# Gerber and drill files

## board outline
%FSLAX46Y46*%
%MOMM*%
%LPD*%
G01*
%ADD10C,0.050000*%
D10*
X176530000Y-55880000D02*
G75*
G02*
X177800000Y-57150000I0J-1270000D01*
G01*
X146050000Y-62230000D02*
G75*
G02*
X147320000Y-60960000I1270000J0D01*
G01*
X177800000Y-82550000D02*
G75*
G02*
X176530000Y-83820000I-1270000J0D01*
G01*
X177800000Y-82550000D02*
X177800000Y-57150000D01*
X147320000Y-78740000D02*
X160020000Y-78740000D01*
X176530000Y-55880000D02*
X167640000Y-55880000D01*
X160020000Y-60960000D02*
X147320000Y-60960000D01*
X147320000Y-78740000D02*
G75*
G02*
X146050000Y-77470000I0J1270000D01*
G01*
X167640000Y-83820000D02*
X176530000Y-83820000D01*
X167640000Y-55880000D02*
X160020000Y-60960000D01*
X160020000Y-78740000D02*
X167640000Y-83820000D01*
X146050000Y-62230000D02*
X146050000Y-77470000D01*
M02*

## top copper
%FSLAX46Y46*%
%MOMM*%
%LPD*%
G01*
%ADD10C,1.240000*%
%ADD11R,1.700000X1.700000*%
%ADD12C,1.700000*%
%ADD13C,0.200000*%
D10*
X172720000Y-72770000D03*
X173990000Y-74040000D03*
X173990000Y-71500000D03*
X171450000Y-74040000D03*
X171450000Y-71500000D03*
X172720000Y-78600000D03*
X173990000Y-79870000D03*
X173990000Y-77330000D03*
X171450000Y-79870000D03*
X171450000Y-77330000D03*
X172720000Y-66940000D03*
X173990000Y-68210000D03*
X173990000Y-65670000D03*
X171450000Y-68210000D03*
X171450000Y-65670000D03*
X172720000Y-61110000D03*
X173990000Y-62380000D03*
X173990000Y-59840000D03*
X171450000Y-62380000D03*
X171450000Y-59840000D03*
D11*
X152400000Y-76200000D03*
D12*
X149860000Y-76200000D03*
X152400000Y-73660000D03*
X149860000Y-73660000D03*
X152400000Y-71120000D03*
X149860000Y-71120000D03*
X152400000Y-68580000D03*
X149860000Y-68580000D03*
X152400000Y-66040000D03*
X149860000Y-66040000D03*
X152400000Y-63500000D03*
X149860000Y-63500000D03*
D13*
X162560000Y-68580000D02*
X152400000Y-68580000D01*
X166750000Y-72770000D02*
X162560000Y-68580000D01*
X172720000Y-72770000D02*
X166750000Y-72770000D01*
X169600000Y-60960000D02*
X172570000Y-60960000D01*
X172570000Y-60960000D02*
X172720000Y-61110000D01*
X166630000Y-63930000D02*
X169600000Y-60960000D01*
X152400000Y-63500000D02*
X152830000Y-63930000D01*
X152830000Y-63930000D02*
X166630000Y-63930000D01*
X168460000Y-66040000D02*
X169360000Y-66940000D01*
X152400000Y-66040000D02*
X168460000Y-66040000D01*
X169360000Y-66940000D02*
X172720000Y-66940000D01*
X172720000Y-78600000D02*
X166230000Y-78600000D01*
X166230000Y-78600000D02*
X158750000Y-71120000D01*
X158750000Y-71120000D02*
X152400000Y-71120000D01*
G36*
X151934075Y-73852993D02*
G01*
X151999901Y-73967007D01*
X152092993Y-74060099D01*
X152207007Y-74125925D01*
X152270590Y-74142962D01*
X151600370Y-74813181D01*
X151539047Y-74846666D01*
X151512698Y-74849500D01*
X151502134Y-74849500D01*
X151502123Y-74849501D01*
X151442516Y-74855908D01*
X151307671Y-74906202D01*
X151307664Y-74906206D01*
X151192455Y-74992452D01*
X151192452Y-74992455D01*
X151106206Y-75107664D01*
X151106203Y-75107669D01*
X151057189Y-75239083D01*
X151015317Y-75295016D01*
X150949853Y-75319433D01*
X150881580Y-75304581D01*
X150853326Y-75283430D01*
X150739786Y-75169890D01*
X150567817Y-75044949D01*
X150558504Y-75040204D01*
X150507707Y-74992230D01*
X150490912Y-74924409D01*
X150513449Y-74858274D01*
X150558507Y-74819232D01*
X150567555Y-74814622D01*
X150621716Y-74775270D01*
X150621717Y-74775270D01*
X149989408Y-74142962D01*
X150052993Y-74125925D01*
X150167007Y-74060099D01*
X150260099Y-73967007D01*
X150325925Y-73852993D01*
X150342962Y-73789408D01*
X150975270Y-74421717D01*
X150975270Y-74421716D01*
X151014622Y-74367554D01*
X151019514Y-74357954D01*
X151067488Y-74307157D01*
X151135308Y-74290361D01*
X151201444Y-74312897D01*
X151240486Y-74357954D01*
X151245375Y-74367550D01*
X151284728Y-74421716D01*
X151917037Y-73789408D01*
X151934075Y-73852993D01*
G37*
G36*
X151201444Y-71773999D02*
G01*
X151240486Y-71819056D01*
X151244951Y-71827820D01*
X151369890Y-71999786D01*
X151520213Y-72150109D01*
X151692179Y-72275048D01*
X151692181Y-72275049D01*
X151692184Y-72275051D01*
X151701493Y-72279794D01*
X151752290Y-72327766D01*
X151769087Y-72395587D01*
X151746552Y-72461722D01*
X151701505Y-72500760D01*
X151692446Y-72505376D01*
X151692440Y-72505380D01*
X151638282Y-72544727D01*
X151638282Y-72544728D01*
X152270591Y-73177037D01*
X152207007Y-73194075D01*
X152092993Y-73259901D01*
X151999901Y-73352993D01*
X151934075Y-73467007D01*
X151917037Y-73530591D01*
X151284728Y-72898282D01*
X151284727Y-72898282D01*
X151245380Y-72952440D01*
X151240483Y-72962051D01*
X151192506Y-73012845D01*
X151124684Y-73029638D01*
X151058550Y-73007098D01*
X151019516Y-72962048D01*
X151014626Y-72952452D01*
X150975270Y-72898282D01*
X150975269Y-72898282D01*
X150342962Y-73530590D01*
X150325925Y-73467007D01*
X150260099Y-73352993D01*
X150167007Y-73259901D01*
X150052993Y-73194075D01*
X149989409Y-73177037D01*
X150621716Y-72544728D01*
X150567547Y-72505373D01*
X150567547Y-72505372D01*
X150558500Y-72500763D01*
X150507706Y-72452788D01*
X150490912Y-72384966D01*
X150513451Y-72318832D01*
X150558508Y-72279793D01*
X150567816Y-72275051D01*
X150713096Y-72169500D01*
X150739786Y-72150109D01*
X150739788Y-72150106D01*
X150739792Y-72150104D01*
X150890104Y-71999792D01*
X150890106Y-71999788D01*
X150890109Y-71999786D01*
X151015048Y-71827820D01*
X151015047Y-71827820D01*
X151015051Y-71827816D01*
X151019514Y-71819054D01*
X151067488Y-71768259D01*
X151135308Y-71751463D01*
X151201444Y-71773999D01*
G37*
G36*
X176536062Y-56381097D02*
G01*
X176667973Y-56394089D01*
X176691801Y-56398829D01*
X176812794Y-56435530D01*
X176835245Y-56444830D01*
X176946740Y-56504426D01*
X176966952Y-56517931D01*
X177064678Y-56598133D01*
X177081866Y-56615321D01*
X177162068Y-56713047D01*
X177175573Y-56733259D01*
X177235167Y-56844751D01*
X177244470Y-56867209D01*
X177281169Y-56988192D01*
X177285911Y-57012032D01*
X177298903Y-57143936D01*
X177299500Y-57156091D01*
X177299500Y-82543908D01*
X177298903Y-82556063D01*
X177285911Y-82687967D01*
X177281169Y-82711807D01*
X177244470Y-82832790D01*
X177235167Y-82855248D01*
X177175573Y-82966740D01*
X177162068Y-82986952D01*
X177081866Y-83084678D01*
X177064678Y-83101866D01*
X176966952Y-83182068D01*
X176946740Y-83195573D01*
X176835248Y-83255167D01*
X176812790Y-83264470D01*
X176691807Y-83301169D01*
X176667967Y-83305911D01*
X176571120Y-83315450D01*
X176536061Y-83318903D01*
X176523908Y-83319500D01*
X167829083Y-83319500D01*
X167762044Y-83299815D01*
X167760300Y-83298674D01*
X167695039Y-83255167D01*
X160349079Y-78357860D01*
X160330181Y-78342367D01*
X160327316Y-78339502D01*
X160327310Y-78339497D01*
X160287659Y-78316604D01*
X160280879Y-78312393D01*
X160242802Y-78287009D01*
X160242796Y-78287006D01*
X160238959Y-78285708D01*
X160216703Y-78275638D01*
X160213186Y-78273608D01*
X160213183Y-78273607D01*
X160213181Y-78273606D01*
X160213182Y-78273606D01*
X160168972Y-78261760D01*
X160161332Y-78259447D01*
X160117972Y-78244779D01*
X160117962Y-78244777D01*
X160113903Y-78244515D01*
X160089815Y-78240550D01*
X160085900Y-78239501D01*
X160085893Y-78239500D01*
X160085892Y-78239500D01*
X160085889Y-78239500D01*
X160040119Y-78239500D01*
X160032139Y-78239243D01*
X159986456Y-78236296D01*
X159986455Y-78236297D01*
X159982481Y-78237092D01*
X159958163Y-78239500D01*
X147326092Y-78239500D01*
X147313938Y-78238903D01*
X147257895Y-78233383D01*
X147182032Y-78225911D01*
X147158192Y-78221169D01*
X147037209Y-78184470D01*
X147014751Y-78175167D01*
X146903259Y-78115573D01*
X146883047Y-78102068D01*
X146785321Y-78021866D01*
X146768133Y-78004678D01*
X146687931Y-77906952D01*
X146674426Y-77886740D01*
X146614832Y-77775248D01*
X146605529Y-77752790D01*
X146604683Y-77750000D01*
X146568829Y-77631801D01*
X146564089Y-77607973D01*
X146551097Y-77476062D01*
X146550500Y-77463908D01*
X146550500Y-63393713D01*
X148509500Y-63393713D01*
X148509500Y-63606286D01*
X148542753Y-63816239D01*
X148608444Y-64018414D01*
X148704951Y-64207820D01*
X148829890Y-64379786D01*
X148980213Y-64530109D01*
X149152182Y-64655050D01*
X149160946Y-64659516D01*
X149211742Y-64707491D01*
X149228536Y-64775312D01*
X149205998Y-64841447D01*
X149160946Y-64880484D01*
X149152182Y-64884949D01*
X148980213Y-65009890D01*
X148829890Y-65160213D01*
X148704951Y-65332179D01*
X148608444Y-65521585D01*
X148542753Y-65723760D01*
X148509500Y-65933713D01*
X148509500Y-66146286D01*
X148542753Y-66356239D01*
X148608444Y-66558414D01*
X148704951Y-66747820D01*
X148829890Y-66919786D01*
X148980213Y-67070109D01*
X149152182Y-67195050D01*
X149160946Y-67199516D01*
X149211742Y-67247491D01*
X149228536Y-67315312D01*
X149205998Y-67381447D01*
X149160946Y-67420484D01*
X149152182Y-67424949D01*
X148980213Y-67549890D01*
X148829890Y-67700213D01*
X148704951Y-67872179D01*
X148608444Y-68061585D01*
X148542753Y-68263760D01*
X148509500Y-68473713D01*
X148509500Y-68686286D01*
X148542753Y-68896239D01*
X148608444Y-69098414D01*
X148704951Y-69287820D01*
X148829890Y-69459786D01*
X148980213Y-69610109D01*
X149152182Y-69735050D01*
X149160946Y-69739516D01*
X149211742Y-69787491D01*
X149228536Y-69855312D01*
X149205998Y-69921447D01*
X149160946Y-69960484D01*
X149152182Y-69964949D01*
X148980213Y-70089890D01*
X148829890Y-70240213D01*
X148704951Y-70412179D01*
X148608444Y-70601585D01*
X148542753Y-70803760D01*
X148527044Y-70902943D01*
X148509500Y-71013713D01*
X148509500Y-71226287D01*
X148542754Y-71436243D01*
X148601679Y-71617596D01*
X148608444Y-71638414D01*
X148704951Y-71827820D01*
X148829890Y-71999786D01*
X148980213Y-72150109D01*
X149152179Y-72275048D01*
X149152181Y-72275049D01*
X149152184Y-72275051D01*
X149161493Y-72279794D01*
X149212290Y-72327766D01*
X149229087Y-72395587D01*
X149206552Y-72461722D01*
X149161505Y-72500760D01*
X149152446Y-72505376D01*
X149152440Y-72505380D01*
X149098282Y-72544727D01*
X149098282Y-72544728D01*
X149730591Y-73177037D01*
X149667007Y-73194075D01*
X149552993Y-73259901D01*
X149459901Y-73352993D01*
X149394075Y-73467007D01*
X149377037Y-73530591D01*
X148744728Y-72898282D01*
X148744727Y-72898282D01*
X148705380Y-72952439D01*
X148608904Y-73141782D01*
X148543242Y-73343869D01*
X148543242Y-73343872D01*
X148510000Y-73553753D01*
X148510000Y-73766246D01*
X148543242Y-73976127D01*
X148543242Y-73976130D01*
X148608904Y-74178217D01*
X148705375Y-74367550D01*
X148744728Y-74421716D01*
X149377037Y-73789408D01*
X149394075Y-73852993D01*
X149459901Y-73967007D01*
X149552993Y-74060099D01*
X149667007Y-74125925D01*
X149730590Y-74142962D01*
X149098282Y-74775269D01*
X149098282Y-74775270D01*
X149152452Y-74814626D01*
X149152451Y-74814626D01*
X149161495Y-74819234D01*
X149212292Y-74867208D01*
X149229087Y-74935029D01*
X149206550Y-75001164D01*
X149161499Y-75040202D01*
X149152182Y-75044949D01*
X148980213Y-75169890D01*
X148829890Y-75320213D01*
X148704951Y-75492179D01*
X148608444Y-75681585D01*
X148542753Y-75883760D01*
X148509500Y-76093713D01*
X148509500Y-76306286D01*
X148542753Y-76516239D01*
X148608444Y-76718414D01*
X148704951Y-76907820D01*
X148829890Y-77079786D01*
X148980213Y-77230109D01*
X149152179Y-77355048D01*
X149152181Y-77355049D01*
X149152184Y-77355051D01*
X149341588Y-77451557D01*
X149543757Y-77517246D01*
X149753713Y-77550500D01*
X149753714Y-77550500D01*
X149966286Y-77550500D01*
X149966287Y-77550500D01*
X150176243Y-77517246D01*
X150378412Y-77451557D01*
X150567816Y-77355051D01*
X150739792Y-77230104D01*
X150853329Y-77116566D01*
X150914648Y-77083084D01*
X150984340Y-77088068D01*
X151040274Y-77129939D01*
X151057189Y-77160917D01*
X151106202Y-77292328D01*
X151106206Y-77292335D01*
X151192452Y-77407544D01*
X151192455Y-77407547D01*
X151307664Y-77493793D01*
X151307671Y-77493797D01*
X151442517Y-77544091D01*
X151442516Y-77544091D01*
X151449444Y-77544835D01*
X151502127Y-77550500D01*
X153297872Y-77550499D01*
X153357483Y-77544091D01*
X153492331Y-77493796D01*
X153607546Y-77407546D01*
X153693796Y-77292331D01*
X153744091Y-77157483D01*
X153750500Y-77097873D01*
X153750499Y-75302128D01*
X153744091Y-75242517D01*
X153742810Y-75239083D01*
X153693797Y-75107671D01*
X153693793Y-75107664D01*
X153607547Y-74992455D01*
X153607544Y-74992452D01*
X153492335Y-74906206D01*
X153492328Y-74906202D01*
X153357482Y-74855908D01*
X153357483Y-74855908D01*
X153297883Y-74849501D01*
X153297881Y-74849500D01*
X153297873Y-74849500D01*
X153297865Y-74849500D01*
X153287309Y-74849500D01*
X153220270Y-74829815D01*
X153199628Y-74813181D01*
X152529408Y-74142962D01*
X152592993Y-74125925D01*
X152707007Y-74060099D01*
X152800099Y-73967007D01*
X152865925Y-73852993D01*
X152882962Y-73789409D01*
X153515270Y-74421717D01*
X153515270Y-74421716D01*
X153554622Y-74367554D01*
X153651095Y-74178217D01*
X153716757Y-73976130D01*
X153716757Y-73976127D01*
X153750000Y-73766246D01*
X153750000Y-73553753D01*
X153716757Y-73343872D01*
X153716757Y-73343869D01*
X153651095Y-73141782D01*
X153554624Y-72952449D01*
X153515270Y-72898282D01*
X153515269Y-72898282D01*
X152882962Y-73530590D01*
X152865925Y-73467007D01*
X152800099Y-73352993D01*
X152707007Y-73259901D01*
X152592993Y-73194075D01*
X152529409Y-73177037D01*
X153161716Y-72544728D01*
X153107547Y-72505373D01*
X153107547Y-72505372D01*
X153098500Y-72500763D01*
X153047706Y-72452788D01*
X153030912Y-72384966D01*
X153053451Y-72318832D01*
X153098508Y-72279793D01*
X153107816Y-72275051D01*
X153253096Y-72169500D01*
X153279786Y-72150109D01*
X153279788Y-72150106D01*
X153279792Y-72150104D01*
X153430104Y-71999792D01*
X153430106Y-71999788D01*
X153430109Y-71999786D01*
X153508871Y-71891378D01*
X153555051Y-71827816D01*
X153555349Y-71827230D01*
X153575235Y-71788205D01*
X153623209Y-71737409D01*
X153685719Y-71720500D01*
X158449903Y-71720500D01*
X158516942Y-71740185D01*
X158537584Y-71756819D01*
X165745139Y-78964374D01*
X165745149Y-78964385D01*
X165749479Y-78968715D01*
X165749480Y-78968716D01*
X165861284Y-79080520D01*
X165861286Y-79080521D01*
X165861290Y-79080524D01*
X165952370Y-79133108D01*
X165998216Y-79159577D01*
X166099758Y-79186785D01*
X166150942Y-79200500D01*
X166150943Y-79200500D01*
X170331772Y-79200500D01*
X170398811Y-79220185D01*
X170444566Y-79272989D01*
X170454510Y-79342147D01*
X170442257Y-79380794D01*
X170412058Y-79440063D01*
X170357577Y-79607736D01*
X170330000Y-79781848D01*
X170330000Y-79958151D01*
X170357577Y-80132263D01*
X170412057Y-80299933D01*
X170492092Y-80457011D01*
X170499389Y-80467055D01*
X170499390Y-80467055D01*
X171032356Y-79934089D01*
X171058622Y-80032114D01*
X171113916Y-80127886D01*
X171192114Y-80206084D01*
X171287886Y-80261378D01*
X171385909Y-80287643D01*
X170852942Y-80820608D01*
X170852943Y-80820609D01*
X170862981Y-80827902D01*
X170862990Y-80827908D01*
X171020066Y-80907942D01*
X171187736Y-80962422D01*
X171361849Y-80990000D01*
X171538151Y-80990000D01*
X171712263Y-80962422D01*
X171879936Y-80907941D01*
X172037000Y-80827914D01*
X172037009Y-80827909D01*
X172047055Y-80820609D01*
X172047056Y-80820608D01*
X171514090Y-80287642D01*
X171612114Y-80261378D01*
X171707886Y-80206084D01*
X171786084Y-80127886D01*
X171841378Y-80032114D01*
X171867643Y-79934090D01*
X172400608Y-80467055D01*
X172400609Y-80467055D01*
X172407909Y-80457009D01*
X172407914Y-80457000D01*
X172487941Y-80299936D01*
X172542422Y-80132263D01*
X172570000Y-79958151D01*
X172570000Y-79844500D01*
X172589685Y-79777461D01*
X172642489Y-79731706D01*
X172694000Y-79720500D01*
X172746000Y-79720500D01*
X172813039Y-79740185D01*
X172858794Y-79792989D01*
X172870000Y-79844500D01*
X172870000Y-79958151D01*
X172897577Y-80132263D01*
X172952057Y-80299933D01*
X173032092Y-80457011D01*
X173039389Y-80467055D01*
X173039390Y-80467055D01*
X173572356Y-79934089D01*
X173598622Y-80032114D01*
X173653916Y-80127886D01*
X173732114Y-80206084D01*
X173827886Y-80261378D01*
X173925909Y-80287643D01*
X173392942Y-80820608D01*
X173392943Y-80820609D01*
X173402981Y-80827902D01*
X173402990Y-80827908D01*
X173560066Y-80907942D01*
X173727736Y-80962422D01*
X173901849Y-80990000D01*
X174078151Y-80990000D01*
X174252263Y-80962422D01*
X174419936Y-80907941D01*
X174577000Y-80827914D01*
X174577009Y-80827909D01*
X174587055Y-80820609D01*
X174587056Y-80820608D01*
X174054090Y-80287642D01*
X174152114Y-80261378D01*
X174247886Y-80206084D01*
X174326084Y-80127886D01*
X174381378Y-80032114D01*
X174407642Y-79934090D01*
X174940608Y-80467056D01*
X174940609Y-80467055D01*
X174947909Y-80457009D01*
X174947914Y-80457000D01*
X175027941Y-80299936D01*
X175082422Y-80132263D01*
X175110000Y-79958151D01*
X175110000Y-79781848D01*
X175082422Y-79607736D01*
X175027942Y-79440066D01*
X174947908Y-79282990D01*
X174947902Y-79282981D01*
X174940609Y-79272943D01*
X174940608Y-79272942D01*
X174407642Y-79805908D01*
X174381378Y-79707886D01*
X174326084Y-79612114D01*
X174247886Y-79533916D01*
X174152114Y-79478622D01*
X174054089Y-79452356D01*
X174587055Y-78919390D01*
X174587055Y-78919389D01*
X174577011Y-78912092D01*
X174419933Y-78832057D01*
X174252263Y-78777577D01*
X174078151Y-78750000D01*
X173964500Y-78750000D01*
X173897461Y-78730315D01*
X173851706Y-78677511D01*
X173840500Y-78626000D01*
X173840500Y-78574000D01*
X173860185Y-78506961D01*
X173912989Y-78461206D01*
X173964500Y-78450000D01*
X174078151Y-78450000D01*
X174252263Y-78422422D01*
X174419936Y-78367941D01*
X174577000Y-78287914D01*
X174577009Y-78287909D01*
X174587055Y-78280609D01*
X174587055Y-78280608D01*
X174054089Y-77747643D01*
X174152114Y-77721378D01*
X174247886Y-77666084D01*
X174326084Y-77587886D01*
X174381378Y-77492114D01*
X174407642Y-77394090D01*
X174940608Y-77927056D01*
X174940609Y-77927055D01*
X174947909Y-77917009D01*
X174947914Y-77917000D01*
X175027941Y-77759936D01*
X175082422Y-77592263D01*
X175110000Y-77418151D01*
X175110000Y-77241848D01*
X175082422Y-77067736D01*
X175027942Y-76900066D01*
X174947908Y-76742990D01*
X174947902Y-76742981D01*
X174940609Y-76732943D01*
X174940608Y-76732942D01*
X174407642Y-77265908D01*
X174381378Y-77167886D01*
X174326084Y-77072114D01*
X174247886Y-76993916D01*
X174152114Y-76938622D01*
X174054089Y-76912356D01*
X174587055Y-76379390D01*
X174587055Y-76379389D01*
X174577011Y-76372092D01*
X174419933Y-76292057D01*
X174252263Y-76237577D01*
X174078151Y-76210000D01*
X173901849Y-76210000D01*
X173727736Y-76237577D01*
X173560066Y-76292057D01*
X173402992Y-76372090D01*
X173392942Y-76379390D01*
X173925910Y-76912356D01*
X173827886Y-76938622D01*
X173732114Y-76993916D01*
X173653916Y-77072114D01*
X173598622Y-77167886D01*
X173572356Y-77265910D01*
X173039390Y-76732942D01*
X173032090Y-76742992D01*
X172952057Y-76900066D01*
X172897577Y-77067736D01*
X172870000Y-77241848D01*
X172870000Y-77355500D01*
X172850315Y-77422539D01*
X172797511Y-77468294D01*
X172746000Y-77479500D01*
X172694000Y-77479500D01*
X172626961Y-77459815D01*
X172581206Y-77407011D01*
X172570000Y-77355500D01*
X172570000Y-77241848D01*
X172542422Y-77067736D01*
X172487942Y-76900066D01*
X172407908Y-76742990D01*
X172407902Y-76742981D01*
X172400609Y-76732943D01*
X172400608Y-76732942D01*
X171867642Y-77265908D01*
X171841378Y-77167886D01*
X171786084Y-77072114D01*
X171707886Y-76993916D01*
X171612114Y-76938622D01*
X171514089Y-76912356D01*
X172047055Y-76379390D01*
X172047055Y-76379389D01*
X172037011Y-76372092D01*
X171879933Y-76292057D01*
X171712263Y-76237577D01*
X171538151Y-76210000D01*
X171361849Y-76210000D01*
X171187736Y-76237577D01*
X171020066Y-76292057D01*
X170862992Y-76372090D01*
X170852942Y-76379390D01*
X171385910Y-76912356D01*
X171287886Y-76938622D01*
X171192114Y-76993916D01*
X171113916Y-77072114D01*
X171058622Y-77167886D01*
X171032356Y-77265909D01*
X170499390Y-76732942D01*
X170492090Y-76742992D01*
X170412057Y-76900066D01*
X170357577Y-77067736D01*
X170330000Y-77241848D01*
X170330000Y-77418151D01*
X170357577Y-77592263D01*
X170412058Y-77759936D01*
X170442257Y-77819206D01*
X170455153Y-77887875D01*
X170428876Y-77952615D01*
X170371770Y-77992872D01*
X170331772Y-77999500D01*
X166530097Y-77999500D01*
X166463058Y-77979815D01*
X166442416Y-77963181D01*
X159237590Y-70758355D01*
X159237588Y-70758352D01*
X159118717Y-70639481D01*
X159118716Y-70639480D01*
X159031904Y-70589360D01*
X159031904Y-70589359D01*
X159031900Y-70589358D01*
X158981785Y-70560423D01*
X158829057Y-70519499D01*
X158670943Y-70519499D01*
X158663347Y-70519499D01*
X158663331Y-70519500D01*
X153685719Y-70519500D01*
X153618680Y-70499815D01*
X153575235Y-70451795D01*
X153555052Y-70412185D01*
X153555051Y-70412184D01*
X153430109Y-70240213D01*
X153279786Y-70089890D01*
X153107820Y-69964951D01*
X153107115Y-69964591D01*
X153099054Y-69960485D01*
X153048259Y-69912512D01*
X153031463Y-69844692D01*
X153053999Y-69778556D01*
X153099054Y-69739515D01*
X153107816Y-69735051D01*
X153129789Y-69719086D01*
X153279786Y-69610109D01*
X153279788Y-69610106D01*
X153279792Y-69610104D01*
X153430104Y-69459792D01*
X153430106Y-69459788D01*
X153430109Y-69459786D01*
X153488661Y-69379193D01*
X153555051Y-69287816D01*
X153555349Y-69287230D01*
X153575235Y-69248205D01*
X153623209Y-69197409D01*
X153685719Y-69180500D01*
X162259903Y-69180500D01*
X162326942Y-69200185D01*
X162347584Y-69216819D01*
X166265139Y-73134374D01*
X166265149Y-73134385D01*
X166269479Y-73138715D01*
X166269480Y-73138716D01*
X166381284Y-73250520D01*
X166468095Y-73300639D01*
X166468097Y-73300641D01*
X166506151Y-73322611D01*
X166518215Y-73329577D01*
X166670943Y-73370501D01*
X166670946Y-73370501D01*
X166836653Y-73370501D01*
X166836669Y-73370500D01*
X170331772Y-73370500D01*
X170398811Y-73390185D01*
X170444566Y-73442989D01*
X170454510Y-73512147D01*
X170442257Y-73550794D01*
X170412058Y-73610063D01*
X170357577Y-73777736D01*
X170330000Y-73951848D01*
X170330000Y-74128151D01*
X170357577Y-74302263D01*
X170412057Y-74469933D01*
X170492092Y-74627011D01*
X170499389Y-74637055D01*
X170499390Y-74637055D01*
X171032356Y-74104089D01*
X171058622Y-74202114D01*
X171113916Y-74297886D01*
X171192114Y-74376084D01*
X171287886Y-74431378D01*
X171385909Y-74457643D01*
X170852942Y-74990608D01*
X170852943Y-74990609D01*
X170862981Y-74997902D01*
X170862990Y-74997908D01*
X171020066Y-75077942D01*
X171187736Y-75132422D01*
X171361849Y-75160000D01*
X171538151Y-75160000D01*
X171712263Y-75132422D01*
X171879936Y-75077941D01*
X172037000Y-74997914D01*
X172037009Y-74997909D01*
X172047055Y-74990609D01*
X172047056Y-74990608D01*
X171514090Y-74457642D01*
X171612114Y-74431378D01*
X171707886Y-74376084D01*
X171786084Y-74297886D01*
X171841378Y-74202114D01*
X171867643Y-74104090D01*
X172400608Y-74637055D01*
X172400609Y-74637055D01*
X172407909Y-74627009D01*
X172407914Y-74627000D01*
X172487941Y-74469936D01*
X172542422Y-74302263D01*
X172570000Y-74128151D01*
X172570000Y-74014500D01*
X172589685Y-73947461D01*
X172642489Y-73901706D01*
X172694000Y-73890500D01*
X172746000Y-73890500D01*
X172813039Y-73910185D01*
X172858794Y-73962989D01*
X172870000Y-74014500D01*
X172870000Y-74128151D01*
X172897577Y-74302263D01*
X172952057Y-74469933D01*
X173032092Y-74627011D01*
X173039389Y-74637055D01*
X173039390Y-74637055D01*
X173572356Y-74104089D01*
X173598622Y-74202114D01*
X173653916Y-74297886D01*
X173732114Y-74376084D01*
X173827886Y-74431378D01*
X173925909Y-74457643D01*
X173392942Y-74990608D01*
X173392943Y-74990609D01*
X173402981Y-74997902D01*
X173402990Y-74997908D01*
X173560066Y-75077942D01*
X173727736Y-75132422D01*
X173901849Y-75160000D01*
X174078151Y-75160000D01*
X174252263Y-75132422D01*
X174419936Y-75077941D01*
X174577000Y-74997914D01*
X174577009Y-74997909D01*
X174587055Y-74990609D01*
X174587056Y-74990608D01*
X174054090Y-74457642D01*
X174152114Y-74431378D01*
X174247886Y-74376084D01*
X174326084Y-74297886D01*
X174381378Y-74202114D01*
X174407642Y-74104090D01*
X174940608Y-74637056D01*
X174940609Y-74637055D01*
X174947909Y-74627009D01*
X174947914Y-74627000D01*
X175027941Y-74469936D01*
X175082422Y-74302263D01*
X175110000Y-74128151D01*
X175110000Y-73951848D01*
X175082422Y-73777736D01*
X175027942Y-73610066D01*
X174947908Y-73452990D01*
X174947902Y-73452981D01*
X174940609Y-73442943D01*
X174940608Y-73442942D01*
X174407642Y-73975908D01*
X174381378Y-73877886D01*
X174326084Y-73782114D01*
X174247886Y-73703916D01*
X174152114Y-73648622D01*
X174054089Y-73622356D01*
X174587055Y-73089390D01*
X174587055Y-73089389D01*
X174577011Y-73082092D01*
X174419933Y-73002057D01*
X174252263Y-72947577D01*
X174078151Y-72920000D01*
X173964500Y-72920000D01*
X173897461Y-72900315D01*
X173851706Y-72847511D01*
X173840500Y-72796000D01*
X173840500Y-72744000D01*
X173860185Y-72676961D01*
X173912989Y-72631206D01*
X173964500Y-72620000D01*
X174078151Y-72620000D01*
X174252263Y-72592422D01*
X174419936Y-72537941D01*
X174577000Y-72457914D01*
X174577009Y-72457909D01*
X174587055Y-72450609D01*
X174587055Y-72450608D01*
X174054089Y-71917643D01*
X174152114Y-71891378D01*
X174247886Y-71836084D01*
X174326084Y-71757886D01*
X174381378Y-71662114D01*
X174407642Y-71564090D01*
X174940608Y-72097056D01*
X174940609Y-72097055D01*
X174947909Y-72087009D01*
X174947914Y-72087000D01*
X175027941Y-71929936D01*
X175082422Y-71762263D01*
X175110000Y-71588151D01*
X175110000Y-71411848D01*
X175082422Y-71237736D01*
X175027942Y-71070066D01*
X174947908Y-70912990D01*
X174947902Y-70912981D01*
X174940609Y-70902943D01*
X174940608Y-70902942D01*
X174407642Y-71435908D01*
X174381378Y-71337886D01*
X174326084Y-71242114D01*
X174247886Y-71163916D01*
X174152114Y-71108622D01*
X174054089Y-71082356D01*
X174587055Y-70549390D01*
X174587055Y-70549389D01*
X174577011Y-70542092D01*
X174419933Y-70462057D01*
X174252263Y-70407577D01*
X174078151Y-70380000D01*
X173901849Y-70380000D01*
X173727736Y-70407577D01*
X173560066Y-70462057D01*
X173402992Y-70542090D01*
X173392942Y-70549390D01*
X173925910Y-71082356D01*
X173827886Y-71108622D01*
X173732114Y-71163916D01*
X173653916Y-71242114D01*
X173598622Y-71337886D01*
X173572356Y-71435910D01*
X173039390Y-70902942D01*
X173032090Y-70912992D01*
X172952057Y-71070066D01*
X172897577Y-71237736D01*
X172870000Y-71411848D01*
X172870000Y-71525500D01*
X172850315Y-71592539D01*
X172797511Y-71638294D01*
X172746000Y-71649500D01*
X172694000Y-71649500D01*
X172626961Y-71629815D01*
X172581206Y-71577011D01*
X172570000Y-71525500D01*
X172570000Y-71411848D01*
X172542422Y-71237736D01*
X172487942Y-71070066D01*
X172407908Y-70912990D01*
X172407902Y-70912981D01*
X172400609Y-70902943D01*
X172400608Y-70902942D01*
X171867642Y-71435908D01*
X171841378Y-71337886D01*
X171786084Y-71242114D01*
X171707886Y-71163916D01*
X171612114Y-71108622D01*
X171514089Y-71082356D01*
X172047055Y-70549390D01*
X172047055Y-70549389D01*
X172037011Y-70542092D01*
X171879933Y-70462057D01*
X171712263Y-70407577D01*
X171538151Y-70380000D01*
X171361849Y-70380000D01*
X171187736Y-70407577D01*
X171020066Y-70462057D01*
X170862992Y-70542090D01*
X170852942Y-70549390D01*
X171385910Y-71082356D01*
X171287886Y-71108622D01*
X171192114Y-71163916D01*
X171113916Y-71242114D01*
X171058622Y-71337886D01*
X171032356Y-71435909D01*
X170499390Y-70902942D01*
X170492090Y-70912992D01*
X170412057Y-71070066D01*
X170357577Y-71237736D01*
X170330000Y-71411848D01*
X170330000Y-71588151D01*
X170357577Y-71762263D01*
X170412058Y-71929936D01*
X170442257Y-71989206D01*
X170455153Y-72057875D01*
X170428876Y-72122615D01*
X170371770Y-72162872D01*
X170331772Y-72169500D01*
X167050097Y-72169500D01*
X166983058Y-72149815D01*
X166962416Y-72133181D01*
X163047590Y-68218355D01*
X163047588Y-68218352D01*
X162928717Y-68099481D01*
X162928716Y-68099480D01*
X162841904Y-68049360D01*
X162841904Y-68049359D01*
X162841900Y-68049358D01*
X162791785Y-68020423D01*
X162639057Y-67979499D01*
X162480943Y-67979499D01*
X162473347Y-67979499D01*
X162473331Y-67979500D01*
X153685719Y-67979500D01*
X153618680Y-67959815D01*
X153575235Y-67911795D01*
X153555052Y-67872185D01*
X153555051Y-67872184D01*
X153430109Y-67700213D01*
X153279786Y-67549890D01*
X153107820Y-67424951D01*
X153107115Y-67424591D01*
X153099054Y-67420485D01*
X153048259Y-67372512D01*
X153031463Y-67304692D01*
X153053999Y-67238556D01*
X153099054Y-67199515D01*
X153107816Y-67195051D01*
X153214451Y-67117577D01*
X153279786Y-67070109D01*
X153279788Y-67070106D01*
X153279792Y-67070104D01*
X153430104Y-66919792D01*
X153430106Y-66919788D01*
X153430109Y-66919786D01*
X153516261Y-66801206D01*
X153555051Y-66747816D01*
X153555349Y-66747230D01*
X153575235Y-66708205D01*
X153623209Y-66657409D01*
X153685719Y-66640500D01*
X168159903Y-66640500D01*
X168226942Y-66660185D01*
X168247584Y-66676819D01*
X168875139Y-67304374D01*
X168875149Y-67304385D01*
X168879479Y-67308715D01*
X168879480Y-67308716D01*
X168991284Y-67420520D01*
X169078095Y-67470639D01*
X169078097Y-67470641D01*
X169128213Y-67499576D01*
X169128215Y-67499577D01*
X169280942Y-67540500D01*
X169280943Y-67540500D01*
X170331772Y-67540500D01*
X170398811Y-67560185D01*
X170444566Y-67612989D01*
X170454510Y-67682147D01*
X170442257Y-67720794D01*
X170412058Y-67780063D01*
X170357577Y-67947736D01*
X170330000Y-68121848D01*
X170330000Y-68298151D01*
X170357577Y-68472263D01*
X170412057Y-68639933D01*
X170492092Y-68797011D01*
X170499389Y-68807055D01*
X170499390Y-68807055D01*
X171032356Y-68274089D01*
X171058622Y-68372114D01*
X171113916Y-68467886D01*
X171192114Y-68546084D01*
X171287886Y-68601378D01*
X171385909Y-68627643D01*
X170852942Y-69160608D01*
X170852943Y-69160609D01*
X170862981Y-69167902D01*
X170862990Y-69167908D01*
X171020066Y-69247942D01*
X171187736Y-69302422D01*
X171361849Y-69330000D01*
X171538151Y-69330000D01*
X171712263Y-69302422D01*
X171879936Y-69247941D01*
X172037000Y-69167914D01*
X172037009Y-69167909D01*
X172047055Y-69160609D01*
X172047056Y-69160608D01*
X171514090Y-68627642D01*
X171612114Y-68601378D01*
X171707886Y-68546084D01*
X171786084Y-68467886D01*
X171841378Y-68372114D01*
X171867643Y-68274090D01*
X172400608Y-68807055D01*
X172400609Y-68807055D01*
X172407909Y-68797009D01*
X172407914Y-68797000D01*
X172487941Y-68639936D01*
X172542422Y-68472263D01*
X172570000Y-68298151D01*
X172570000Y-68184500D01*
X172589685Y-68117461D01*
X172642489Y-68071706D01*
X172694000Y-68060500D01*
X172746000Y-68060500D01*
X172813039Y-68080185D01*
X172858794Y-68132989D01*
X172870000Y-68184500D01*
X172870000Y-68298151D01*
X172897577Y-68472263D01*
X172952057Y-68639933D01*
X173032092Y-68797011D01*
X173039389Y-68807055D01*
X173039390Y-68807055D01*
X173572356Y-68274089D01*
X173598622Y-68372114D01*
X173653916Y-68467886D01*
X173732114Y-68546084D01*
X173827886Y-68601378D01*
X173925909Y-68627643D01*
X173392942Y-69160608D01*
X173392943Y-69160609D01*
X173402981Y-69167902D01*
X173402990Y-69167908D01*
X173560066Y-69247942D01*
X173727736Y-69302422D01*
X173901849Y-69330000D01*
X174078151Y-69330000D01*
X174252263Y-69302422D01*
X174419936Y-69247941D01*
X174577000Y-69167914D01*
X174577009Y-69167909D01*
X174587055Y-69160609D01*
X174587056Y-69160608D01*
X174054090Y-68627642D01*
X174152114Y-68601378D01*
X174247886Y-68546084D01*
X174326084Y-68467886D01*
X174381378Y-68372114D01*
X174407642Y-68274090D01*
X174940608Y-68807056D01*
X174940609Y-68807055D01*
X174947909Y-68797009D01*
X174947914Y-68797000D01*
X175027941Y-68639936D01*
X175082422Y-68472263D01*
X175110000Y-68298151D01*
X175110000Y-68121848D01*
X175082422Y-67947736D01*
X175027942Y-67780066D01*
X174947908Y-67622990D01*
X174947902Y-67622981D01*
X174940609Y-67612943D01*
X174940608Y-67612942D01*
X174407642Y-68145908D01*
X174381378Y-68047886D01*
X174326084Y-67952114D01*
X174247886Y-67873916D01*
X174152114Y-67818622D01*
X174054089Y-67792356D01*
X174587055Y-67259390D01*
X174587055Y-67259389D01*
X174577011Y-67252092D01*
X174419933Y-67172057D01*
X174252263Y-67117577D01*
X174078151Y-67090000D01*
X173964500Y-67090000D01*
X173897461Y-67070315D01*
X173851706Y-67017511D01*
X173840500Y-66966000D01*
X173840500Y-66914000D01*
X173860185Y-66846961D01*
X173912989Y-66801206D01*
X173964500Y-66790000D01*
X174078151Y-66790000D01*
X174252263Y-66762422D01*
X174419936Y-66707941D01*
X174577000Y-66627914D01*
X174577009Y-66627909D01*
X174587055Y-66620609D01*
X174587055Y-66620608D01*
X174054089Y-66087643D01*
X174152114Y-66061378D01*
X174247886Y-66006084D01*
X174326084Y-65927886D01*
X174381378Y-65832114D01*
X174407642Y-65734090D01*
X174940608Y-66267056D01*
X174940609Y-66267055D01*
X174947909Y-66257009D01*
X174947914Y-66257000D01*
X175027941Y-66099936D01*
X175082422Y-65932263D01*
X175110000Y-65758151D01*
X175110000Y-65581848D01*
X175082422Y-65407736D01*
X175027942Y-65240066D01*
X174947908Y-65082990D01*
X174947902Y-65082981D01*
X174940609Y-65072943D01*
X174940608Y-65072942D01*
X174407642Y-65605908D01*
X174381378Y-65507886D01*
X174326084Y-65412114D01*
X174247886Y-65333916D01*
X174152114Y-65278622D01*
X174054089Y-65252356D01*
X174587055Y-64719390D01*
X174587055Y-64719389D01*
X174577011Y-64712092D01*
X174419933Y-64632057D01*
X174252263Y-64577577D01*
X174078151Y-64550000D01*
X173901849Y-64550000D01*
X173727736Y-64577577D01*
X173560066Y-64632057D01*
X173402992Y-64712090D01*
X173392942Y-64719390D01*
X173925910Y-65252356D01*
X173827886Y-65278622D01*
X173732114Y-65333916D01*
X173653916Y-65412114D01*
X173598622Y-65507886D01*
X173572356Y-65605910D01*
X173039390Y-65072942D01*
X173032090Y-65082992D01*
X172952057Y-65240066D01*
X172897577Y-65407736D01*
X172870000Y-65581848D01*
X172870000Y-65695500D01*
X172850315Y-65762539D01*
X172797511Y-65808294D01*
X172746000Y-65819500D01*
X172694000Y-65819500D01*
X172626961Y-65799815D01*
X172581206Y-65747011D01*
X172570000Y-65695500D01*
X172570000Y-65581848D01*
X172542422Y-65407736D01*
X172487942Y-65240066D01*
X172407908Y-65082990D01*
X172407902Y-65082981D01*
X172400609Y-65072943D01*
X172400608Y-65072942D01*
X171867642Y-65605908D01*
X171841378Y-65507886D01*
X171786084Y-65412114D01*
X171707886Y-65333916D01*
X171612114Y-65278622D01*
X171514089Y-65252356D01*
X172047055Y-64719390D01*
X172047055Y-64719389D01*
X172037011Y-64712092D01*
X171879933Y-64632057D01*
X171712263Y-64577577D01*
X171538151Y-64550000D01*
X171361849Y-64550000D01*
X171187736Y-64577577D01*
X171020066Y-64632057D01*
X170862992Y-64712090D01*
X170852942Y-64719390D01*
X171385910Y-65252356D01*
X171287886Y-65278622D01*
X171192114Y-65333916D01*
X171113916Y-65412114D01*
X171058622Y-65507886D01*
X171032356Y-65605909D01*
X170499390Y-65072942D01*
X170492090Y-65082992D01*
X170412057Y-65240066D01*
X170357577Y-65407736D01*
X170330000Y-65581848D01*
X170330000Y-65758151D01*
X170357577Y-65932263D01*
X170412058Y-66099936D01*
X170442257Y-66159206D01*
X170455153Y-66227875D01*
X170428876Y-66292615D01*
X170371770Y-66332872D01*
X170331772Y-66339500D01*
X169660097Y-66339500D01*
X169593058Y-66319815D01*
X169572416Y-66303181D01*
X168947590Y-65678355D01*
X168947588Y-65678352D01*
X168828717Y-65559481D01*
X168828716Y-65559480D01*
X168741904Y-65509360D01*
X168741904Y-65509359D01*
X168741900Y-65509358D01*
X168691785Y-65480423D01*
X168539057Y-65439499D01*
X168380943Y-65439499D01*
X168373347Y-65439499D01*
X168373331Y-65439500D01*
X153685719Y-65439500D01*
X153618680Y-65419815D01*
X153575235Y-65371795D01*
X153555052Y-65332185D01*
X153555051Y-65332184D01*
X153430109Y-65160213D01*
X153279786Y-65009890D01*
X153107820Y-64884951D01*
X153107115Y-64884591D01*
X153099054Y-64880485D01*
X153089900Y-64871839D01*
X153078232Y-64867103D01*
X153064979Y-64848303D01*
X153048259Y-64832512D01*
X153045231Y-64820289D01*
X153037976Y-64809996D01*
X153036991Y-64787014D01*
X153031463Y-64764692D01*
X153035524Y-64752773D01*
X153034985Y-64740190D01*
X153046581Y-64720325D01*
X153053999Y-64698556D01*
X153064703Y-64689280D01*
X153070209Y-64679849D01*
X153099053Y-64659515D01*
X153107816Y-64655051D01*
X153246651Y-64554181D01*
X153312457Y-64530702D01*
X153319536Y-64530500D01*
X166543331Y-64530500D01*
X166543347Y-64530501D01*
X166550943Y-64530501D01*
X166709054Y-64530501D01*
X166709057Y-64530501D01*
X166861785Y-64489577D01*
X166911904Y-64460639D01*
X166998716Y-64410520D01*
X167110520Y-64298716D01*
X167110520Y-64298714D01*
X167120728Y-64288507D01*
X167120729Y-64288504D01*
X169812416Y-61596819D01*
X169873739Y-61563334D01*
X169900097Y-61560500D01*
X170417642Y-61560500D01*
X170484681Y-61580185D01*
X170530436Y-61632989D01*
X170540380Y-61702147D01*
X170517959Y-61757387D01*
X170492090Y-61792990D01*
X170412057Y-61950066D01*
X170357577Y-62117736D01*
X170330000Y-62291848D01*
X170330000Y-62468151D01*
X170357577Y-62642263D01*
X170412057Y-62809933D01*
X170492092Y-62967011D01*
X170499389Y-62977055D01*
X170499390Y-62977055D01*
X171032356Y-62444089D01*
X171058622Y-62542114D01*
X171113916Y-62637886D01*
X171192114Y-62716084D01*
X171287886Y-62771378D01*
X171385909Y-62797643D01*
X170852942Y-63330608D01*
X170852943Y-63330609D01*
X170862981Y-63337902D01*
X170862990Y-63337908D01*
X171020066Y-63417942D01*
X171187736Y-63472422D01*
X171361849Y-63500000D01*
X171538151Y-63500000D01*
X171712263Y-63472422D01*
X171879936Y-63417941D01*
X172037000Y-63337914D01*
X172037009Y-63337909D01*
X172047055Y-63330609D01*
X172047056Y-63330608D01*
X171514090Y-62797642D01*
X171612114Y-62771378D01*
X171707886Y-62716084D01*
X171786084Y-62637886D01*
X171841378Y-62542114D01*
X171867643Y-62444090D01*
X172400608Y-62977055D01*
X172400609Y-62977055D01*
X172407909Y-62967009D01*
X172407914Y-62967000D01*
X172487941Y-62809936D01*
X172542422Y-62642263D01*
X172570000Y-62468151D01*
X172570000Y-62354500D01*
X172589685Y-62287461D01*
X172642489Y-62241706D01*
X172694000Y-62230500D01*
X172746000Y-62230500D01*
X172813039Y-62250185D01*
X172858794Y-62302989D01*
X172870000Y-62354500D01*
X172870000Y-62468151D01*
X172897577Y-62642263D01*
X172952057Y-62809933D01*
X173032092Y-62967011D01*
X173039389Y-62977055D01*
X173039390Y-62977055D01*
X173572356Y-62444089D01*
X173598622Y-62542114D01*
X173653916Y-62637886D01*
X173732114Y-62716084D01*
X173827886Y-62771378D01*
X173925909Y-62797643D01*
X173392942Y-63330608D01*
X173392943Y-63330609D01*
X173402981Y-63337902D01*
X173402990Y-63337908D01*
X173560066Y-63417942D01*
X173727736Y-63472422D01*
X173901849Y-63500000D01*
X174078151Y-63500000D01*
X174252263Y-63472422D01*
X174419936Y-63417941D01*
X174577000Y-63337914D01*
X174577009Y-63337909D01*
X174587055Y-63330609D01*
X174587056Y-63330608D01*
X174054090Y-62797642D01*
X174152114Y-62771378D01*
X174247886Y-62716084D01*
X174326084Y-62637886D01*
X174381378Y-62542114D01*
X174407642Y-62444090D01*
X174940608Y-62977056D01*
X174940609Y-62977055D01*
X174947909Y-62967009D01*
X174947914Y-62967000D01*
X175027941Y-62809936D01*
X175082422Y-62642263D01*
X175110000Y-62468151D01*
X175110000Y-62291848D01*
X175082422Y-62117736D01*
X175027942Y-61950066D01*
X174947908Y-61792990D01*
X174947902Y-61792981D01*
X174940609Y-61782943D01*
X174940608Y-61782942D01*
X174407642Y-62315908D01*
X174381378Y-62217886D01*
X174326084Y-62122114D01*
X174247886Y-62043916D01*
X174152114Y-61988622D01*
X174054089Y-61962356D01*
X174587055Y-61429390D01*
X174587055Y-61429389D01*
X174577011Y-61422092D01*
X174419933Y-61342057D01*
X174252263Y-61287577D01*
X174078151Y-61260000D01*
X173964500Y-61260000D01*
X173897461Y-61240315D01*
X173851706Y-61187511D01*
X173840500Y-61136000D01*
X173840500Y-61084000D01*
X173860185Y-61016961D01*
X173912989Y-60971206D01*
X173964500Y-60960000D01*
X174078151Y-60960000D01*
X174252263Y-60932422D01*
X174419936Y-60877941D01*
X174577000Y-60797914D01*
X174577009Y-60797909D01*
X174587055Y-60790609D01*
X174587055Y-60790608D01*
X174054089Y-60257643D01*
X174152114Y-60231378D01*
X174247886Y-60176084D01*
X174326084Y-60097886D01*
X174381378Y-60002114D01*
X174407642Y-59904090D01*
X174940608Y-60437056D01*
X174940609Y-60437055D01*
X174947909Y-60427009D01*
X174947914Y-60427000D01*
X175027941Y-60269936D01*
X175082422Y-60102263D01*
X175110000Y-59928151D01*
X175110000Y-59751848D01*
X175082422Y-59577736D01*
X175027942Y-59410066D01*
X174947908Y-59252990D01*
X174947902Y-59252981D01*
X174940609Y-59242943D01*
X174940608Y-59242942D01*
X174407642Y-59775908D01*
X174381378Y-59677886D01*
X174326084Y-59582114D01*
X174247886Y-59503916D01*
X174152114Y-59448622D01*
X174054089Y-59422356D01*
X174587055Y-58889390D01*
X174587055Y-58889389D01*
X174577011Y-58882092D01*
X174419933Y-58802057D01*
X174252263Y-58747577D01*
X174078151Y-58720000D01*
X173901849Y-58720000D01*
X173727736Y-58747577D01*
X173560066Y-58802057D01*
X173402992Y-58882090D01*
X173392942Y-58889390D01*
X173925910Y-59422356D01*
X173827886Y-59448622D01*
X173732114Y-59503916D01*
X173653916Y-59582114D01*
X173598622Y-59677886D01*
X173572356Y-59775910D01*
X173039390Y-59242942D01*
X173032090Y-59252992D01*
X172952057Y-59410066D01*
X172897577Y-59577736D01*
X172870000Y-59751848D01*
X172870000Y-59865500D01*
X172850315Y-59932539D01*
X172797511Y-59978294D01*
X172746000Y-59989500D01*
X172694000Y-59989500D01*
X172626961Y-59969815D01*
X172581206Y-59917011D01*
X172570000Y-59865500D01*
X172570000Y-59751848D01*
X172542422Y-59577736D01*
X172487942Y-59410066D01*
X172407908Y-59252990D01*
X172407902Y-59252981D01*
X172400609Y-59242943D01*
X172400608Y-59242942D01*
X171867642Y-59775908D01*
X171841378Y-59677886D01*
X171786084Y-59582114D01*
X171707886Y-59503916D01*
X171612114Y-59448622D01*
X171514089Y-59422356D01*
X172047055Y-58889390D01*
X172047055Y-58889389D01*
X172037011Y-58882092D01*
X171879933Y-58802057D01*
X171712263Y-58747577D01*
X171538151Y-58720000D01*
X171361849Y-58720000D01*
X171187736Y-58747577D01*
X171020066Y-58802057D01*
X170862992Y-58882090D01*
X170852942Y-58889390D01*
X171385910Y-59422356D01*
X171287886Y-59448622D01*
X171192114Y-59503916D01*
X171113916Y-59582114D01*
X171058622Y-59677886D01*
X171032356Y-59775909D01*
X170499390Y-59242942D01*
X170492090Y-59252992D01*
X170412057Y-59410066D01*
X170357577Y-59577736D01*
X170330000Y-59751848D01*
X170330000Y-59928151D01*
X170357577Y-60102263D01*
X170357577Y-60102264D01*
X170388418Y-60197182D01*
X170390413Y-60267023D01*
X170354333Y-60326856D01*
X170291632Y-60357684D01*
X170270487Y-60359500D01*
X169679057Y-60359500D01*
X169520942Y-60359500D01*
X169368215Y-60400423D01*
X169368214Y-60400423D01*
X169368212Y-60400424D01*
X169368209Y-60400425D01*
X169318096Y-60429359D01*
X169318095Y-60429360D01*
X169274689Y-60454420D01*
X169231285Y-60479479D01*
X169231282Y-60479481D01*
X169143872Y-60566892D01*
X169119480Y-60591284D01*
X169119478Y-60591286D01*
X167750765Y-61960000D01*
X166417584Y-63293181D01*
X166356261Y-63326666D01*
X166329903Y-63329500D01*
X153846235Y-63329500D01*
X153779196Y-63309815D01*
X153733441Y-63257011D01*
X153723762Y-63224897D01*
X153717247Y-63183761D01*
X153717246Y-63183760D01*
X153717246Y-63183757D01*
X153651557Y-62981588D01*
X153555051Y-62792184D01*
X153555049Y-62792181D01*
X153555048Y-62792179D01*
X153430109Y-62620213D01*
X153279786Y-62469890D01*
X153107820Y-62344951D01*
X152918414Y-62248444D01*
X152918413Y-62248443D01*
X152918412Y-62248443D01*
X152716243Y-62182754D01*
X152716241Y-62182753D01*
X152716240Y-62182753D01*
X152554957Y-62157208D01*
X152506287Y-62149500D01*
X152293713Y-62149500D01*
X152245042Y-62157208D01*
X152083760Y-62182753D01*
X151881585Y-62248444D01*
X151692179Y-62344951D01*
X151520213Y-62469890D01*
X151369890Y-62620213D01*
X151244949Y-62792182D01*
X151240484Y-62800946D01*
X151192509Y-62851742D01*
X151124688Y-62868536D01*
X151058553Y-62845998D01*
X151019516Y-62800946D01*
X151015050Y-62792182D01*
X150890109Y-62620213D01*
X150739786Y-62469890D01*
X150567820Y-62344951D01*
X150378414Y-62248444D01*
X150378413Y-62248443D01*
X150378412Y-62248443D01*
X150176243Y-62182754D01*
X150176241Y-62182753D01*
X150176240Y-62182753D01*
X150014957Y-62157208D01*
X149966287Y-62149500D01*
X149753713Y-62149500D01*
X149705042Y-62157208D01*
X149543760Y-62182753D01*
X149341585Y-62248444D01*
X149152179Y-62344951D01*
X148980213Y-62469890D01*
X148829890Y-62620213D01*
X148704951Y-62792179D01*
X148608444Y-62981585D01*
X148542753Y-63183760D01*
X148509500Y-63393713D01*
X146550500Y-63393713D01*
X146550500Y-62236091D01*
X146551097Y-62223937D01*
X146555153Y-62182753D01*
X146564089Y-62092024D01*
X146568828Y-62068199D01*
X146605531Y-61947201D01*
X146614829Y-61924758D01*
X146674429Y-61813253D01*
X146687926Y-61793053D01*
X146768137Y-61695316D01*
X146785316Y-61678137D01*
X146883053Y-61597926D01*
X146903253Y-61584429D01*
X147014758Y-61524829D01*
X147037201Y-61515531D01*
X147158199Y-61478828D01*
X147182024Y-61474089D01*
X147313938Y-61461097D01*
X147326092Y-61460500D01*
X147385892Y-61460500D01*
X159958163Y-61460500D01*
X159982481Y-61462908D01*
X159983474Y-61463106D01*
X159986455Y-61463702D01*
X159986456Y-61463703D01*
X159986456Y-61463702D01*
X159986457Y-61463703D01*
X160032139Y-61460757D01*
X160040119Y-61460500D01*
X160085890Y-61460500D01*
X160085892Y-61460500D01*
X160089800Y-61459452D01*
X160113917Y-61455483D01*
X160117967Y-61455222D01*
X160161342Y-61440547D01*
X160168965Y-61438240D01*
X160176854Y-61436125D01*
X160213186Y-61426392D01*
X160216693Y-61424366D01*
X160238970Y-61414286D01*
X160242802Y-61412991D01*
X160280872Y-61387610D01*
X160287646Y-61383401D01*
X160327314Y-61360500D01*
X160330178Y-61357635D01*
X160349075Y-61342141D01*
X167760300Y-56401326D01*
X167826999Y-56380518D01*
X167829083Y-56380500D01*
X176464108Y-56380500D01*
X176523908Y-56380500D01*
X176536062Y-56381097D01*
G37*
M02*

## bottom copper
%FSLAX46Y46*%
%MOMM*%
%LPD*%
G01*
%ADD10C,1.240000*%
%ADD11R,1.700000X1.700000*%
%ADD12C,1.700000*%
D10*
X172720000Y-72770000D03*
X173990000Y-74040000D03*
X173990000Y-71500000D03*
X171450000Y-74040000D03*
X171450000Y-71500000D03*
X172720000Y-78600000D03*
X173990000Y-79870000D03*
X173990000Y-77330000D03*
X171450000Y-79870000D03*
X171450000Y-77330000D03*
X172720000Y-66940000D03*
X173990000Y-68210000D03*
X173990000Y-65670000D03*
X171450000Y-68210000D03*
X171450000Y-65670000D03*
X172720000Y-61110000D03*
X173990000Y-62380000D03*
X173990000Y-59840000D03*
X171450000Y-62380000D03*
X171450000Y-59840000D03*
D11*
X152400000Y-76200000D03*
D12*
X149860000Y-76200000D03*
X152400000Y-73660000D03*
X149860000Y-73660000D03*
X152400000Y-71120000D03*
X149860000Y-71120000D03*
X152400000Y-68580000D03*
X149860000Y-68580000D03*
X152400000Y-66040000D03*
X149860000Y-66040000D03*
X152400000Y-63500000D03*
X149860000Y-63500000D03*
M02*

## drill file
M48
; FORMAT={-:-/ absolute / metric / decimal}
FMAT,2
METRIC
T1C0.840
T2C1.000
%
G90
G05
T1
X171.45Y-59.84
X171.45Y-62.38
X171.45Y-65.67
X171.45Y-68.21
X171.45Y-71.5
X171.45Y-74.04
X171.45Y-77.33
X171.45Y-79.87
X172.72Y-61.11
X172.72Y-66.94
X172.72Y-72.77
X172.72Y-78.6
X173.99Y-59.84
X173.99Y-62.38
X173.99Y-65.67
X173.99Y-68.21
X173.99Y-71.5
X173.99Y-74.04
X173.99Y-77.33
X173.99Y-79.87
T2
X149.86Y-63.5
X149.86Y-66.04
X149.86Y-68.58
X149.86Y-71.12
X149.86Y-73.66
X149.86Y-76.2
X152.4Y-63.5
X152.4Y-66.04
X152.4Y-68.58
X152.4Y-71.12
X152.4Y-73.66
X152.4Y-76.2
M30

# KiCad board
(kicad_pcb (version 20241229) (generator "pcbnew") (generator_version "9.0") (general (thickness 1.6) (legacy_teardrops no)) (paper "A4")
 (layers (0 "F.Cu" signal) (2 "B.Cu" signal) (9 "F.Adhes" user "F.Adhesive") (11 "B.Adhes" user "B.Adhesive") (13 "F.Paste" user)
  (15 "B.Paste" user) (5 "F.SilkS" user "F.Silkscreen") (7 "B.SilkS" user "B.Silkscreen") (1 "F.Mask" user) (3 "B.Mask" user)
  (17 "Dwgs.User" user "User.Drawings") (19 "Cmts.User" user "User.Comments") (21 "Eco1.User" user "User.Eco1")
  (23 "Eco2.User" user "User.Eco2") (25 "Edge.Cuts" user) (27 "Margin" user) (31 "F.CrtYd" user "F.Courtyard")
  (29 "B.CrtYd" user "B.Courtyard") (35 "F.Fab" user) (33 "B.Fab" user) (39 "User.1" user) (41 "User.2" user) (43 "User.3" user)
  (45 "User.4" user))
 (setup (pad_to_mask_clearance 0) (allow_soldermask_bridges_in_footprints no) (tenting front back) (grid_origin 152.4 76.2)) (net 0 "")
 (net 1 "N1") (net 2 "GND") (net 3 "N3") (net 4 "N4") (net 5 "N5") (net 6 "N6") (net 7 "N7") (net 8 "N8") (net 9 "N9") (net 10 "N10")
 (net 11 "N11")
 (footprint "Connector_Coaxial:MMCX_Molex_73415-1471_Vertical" (layer "F.Cu") (at 172.72 72.77 180)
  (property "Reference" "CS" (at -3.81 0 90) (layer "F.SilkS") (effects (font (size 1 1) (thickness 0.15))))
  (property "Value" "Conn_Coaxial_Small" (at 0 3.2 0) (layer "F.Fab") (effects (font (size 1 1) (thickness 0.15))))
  (pad "1" thru_hole circle (at 0 0 180) (size 1.24 1.24) (drill 0.84) (layers "*.Cu" "*.Mask") (remove_unused_layers no) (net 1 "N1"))
  (pad "2" thru_hole circle (at -1.27 -1.27 180) (size 1.24 1.24) (drill 0.84) (layers "*.Cu" "*.Mask") (remove_unused_layers no)
   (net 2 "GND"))
  (pad "2" thru_hole circle (at -1.27 1.27 180) (size 1.24 1.24) (drill 0.84) (layers "*.Cu" "*.Mask") (remove_unused_layers no)
   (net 2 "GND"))
  (pad "2" thru_hole circle (at 1.27 -1.27 180) (size 1.24 1.24) (drill 0.84) (layers "*.Cu" "*.Mask") (remove_unused_layers no)
   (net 2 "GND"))
  (pad "2" thru_hole circle (at 1.27 1.27 180) (size 1.24 1.24) (drill 0.84) (layers "*.Cu" "*.Mask") (remove_unused_layers no)
   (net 2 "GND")))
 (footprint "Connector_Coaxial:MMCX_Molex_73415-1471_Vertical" (layer "F.Cu") (at 172.72 78.6 180)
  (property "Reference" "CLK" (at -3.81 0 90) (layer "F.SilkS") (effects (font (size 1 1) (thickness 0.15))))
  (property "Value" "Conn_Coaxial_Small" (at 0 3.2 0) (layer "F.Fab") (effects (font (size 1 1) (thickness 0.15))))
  (pad "1" thru_hole circle (at 0 0 180) (size 1.24 1.24) (drill 0.84) (layers "*.Cu" "*.Mask") (remove_unused_layers no) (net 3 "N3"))
  (pad "2" thru_hole circle (at -1.27 -1.27 180) (size 1.24 1.24) (drill 0.84) (layers "*.Cu" "*.Mask") (remove_unused_layers no)
   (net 2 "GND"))
  (pad "2" thru_hole circle (at -1.27 1.27 180) (size 1.24 1.24) (drill 0.84) (layers "*.Cu" "*.Mask") (remove_unused_layers no)
   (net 2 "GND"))
  (pad "2" thru_hole circle (at 1.27 -1.27 180) (size 1.24 1.24) (drill 0.84) (layers "*.Cu" "*.Mask") (remove_unused_layers no)
   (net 2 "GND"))
  (pad "2" thru_hole circle (at 1.27 1.27 180) (size 1.24 1.24) (drill 0.84) (layers "*.Cu" "*.Mask") (remove_unused_layers no)
   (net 2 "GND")))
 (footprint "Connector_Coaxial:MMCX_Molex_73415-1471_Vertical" (layer "F.Cu") (at 172.72 66.94 180)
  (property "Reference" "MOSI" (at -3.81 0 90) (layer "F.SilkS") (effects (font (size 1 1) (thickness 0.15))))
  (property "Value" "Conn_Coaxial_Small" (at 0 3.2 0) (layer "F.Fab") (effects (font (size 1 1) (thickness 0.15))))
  (pad "1" thru_hole circle (at 0 0 180) (size 1.24 1.24) (drill 0.84) (layers "*.Cu" "*.Mask") (remove_unused_layers no) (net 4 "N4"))
  (pad "2" thru_hole circle (at -1.27 -1.27 180) (size 1.24 1.24) (drill 0.84) (layers "*.Cu" "*.Mask") (remove_unused_layers no)
   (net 2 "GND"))
  (pad "2" thru_hole circle (at -1.27 1.27 180) (size 1.24 1.24) (drill 0.84) (layers "*.Cu" "*.Mask") (remove_unused_layers no)
   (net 2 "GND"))
  (pad "2" thru_hole circle (at 1.27 -1.27 180) (size 1.24 1.24) (drill 0.84) (layers "*.Cu" "*.Mask") (remove_unused_layers no)
   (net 2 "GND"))
  (pad "2" thru_hole circle (at 1.27 1.27 180) (size 1.24 1.24) (drill 0.84) (layers "*.Cu" "*.Mask") (remove_unused_layers no)
   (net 2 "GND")))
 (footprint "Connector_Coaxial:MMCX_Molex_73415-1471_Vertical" (layer "F.Cu") (at 172.72 61.11 180)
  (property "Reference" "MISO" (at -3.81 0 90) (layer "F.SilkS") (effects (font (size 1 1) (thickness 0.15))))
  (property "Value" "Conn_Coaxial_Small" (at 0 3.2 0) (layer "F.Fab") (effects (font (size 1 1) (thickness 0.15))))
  (pad "1" thru_hole circle (at 0 0 180) (size 1.24 1.24) (drill 0.84) (layers "*.Cu" "*.Mask") (remove_unused_layers no) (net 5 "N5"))
  (pad "2" thru_hole circle (at -1.27 -1.27 180) (size 1.24 1.24) (drill 0.84) (layers "*.Cu" "*.Mask") (remove_unused_layers no)
   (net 2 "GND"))
  (pad "2" thru_hole circle (at -1.27 1.27 180) (size 1.24 1.24) (drill 0.84) (layers "*.Cu" "*.Mask") (remove_unused_layers no)
   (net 2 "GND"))
  (pad "2" thru_hole circle (at 1.27 -1.27 180) (size 1.24 1.24) (drill 0.84) (layers "*.Cu" "*.Mask") (remove_unused_layers no)
   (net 2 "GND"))
  (pad "2" thru_hole circle (at 1.27 1.27 180) (size 1.24 1.24) (drill 0.84) (layers "*.Cu" "*.Mask") (remove_unused_layers no)
   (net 2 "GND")))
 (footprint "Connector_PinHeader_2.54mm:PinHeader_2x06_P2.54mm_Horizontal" (layer "F.Cu") (at 152.4 76.2 180)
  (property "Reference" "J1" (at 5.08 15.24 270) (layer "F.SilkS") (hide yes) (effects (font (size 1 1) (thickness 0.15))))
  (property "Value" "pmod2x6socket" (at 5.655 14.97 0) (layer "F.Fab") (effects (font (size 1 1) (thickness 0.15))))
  (pad "1" thru_hole rect (at 0 0 180) (size 1.7 1.7) (drill 1) (layers "*.Cu" "*.Mask") (remove_unused_layers no) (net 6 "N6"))
  (pad "2" thru_hole circle (at 2.54 0 180) (size 1.7 1.7) (drill 1) (layers "*.Cu" "*.Mask") (remove_unused_layers no) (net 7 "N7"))
  (pad "3" thru_hole circle (at 0 2.54 180) (size 1.7 1.7) (drill 1) (layers "*.Cu" "*.Mask") (remove_unused_layers no) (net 2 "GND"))
  (pad "4" thru_hole circle (at 2.54 2.54 180) (size 1.7 1.7) (drill 1) (layers "*.Cu" "*.Mask") (remove_unused_layers no) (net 2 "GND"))
  (pad "5" thru_hole circle (at 0 5.08 180) (size 1.7 1.7) (drill 1) (layers "*.Cu" "*.Mask") (remove_unused_layers no) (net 3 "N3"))
  (pad "6" thru_hole circle (at 2.54 5.08 180) (size 1.7 1.7) (drill 1) (layers "*.Cu" "*.Mask") (remove_unused_layers no) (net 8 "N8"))
  (pad "7" thru_hole circle (at 0 7.62 180) (size 1.7 1.7) (drill 1) (layers "*.Cu" "*.Mask") (remove_unused_layers no) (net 1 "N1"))
  (pad "8" thru_hole circle (at 2.54 7.62 180) (size 1.7 1.7) (drill 1) (layers "*.Cu" "*.Mask") (remove_unused_layers no) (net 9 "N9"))
  (pad "9" thru_hole circle (at 0 10.16 180) (size 1.7 1.7) (drill 1) (layers "*.Cu" "*.Mask") (remove_unused_layers no) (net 4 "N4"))
  (pad "10" thru_hole circle (at 2.54 10.16 180) (size 1.7 1.7) (drill 1) (layers "*.Cu" "*.Mask") (remove_unused_layers no) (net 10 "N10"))
  (pad "11" thru_hole circle (at 0 12.7 180) (size 1.7 1.7) (drill 1) (layers "*.Cu" "*.Mask") (remove_unused_layers no) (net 5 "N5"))
  (pad "12" thru_hole circle (at 2.54 12.7 180) (size 1.7 1.7) (drill 1) (layers "*.Cu" "*.Mask") (remove_unused_layers no) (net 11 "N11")))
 (gr_arc (start 176.53 55.88) (mid 177.428026 56.251974) (end 177.8 57.15) (stroke (width 0.05) (type default)) (layer "Edge.Cuts"))
 (gr_arc (start 146.05 62.23) (mid 146.421974 61.331974) (end 147.32 60.96) (stroke (width 0.05) (type default)) (layer "Edge.Cuts"))
 (gr_arc (start 177.8 82.55) (mid 177.428026 83.448026) (end 176.53 83.82) (stroke (width 0.05) (type default)) (layer "Edge.Cuts"))
 (gr_line (start 177.8 82.55) (end 177.8 57.15) (stroke (width 0.05) (type default)) (layer "Edge.Cuts"))
 (gr_line (start 147.32 78.74) (end 160.02 78.74) (stroke (width 0.05) (type default)) (layer "Edge.Cuts"))
 (gr_line (start 176.53 55.88) (end 167.64 55.88) (stroke (width 0.05) (type default)) (layer "Edge.Cuts"))
 (gr_line (start 160.02 60.96) (end 147.32 60.96) (stroke (width 0.05) (type default)) (layer "Edge.Cuts"))
 (gr_arc (start 147.32 78.74) (mid 146.421974 78.368026) (end 146.05 77.47) (stroke (width 0.05) (type default)) (layer "Edge.Cuts"))
 (gr_line (start 167.64 83.82) (end 176.53 83.82) (stroke (width 0.05) (type default)) (layer "Edge.Cuts"))
 (gr_line (start 167.64 55.88) (end 160.02 60.96) (stroke (width 0.05) (type default)) (layer "Edge.Cuts"))
 (gr_line (start 160.02 78.74) (end 167.64 83.82) (stroke (width 0.05) (type default)) (layer "Edge.Cuts"))
 (gr_line (start 146.05 62.23) (end 146.05 77.47) (stroke (width 0.05) (type default)) (layer "Edge.Cuts"))
 (segment (start 162.56 68.58) (end 152.4 68.58) (width 0.2) (layer "F.Cu") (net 1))
 (segment (start 166.75 72.77) (end 162.56 68.58) (width 0.2) (layer "F.Cu") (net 1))
 (segment (start 172.72 72.77) (end 166.75 72.77) (width 0.2) (layer "F.Cu") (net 1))
 (segment (start 169.6 60.96) (end 172.57 60.96) (width 0.2) (layer "F.Cu") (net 5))
 (segment (start 172.57 60.96) (end 172.72 61.11) (width 0.2) (layer "F.Cu") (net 5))
 (segment (start 166.63 63.93) (end 169.6 60.96) (width 0.2) (layer "F.Cu") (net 5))
 (segment (start 152.4 63.5) (end 152.83 63.93) (width 0.2) (layer "F.Cu") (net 5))
 (segment (start 152.83 63.93) (end 166.63 63.93) (width 0.2) (layer "F.Cu") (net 5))
 (segment (start 168.46 66.04) (end 169.36 66.94) (width 0.2) (layer "F.Cu") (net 4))
 (segment (start 152.4 66.04) (end 168.46 66.04) (width 0.2) (layer "F.Cu") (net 4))
 (segment (start 169.36 66.94) (end 172.72 66.94) (width 0.2) (layer "F.Cu") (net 4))
 (segment (start 172.72 78.6) (end 166.23 78.6) (width 0.2) (layer "F.Cu") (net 3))
 (segment (start 166.23 78.6) (end 158.75 71.12) (width 0.2) (layer "F.Cu") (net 3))
 (segment (start 158.75 71.12) (end 152.4 71.12) (width 0.2) (layer "F.Cu") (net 3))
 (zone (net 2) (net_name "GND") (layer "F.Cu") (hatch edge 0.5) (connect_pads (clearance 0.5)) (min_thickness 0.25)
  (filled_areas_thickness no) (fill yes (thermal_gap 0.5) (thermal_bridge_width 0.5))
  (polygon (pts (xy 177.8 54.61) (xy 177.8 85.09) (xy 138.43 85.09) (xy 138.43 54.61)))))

